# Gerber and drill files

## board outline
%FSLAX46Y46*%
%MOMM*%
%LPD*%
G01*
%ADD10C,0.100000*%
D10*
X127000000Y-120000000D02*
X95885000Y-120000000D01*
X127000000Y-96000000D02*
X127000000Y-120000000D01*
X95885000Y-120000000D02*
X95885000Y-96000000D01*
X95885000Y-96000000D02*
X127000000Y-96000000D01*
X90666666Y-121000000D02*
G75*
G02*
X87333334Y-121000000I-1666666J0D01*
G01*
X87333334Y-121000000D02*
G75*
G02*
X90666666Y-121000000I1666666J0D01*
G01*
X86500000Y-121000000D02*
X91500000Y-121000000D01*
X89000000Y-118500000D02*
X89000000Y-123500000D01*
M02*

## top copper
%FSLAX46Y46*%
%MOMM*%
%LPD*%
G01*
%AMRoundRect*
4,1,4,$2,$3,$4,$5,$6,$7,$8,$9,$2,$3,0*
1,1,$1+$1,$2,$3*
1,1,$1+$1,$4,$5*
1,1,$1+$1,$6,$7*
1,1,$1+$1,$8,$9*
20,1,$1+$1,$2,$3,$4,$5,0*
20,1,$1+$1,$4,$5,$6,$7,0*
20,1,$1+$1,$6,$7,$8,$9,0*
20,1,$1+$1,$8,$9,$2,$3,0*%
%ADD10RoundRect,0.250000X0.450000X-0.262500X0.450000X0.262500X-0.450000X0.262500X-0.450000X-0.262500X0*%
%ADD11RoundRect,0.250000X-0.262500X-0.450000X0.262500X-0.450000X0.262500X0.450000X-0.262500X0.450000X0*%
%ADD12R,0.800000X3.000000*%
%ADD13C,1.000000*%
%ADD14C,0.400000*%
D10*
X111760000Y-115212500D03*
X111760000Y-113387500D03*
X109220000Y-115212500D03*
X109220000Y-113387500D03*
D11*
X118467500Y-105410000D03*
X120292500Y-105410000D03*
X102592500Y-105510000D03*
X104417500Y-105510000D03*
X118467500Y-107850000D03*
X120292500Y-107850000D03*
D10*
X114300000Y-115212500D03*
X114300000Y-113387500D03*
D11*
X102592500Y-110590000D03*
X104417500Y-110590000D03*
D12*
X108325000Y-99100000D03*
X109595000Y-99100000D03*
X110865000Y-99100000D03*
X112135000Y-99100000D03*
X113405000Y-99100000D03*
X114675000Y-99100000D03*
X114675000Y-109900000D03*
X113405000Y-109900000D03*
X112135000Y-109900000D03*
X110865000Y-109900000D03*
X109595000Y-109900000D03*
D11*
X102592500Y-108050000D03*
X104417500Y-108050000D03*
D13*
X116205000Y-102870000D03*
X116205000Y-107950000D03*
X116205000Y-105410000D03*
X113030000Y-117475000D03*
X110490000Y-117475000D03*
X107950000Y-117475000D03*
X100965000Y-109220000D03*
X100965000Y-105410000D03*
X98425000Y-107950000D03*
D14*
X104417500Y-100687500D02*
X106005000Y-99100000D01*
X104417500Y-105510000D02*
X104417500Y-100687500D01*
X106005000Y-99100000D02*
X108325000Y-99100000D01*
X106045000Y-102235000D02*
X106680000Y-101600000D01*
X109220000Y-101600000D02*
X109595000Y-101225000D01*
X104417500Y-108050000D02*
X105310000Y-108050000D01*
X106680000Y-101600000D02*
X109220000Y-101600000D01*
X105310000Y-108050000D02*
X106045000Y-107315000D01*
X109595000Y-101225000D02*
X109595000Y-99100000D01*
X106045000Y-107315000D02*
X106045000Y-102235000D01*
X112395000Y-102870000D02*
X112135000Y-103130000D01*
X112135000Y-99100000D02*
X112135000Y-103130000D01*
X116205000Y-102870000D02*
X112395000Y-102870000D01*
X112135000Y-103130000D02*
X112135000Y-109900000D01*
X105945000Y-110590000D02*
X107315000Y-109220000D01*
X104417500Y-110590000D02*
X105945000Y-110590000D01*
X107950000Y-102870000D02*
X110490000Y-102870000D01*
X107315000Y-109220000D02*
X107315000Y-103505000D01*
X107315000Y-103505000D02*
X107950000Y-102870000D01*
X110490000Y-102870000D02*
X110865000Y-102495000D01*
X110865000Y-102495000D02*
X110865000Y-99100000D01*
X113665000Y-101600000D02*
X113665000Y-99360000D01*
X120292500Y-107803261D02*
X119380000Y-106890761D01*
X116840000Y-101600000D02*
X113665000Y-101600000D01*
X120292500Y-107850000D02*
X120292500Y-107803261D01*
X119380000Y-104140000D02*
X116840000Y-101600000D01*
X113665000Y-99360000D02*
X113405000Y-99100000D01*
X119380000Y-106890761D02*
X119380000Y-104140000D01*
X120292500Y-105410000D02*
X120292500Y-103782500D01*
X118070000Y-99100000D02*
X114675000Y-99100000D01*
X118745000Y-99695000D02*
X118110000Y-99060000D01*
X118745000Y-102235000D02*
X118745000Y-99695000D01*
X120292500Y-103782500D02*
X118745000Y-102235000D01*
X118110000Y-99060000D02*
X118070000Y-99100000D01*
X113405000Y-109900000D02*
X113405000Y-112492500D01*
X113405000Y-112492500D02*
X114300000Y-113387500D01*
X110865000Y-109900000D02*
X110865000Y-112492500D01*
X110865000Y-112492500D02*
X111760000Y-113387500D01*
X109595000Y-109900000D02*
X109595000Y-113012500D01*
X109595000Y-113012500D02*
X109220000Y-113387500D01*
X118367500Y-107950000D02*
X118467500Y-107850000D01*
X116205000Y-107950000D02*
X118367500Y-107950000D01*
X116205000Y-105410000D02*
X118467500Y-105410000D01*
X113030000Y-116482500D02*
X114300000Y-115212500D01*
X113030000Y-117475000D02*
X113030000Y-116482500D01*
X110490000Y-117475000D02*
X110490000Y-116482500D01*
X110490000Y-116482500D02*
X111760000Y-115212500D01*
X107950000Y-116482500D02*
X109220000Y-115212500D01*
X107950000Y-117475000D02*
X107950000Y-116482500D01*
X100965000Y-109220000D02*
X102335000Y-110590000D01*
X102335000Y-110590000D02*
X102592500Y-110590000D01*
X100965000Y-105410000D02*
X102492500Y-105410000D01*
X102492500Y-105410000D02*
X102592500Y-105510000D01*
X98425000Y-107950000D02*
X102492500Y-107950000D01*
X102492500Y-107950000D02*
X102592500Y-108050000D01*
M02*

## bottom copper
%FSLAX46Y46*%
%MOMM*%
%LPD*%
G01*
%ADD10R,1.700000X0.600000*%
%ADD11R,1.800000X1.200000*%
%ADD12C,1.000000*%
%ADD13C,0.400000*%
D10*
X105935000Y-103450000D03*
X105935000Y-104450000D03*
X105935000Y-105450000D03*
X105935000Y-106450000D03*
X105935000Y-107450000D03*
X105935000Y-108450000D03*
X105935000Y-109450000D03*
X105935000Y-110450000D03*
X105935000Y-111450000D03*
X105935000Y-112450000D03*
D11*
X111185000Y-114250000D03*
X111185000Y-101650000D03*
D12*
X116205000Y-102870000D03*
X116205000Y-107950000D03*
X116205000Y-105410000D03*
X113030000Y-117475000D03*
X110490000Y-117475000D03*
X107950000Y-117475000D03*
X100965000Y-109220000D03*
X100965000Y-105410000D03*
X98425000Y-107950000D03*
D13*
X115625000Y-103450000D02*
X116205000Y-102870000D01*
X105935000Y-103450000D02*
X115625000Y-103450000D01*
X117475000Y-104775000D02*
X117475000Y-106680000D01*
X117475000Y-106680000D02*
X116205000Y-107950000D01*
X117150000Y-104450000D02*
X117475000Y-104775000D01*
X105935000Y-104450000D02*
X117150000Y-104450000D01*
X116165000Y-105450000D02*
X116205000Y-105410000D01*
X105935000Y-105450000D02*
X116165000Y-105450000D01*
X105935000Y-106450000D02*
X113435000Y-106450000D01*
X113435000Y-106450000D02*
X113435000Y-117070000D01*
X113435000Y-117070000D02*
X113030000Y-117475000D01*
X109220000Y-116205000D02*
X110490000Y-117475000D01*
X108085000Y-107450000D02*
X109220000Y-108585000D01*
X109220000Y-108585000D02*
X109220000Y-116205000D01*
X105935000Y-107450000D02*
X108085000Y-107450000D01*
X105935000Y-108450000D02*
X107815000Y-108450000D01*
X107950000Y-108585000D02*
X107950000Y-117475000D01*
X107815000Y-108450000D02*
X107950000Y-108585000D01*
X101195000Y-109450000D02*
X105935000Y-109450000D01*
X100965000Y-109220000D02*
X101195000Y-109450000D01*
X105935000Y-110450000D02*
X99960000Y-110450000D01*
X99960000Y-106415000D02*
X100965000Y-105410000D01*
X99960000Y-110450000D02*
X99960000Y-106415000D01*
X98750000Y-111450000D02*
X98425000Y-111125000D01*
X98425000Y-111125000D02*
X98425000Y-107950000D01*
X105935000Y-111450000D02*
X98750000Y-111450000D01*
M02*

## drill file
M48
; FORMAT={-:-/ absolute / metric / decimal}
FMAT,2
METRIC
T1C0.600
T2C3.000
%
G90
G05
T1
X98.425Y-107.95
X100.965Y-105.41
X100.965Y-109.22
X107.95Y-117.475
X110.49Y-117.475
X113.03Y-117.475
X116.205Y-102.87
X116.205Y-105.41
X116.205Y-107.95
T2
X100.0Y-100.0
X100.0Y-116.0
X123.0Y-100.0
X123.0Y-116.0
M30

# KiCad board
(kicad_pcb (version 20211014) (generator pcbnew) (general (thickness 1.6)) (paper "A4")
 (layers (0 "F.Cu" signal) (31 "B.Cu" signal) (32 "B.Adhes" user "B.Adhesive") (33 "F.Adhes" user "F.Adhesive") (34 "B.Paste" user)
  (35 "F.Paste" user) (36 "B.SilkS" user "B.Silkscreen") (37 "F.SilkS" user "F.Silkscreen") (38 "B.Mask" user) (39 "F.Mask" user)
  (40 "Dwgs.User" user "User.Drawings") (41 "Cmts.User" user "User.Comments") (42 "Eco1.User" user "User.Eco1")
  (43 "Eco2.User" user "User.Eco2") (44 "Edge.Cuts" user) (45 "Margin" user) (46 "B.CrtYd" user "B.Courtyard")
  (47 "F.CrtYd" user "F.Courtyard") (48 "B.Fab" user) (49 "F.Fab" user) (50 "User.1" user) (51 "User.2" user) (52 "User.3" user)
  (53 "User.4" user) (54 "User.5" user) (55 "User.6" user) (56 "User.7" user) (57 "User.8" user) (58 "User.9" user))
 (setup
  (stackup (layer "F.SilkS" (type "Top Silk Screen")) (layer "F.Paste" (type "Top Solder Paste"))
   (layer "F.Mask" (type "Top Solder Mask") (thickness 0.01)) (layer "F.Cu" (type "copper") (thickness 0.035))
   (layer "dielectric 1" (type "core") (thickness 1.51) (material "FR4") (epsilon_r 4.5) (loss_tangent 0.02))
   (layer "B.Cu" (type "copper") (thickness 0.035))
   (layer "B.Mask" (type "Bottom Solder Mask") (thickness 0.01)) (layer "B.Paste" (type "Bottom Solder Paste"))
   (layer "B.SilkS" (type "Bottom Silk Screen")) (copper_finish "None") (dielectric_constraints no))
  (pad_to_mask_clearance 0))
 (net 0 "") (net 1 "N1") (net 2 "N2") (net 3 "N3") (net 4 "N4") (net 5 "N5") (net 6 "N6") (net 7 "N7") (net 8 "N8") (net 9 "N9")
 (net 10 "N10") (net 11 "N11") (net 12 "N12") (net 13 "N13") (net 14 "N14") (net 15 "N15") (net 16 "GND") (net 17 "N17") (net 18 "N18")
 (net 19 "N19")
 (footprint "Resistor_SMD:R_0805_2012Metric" (layer "F.Cu") (at 111.76 114.3 90)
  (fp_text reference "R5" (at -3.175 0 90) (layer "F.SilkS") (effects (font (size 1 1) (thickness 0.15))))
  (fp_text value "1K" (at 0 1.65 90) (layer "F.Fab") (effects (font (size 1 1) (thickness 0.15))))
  (pad "1" smd roundrect (at -0.9125 0 90) (size 1.025 1.4) (layers "F.Cu" "F.Paste" "F.Mask") (roundrect_rratio 0.243902) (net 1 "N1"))
  (pad "2" smd roundrect (at 0.9125 0 90) (size 1.025 1.4) (layers "F.Cu" "F.Paste" "F.Mask") (roundrect_rratio 0.243902) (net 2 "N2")))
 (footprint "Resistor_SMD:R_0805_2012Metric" (layer "F.Cu") (at 109.22 114.3 90)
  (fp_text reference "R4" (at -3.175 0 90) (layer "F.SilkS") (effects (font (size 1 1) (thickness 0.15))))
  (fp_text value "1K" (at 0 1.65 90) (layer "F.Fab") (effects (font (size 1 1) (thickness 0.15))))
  (pad "1" smd roundrect (at -0.9125 0 90) (size 1.025 1.4) (layers "F.Cu" "F.Paste" "F.Mask") (roundrect_rratio 0.243902) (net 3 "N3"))
  (pad "2" smd roundrect (at 0.9125 0 90) (size 1.025 1.4) (layers "F.Cu" "F.Paste" "F.Mask") (roundrect_rratio 0.243902) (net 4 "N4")))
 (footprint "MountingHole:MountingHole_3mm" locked (layer "F.Cu") (at 100 100)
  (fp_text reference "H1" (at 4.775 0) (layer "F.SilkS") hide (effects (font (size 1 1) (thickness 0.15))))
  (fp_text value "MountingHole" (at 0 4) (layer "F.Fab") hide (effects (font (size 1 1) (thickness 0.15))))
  (pad "" np_thru_hole circle locked (at 0 0) (size 3 3) (drill 3) (layers *.Cu *.Mask)))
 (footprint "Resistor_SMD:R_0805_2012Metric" (layer "F.Cu") (at 119.38 105.41)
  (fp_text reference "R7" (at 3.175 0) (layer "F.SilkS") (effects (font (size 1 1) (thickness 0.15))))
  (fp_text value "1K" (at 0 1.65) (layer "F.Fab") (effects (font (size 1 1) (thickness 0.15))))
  (pad "1" smd roundrect (at -0.9125 0) (size 1.025 1.4) (layers "F.Cu" "F.Paste" "F.Mask") (roundrect_rratio 0.243902) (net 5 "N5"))
  (pad "2" smd roundrect (at 0.9125 0) (size 1.025 1.4) (layers "F.Cu" "F.Paste" "F.Mask") (roundrect_rratio 0.243902) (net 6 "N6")))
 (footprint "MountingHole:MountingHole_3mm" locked (layer "F.Cu") (at 123 116)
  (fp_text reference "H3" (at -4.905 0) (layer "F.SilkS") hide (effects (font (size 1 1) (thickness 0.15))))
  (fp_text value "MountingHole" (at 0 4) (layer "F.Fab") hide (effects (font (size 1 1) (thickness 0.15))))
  (pad "" np_thru_hole circle locked (at 0 0) (size 3 3) (drill 3) (layers *.Cu *.Mask)))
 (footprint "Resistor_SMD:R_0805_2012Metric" (layer "F.Cu") (at 103.505 105.51)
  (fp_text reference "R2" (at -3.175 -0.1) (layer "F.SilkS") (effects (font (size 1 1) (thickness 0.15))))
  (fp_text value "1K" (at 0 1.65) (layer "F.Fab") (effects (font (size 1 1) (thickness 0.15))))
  (pad "1" smd roundrect (at -0.9125 0) (size 1.025 1.4) (layers "F.Cu" "F.Paste" "F.Mask") (roundrect_rratio 0.243902) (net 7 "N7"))
  (pad "2" smd roundrect (at 0.9125 0) (size 1.025 1.4) (layers "F.Cu" "F.Paste" "F.Mask") (roundrect_rratio 0.243902) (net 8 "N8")))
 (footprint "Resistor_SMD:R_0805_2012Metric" (layer "F.Cu") (at 119.38 107.85)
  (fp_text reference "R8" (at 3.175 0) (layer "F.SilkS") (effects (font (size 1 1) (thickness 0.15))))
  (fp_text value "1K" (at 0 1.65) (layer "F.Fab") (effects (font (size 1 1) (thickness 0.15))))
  (pad "1" smd roundrect (at -0.9125 0) (size 1.025 1.4) (layers "F.Cu" "F.Paste" "F.Mask") (roundrect_rratio 0.243902) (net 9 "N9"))
  (pad "2" smd roundrect (at 0.9125 0) (size 1.025 1.4) (layers "F.Cu" "F.Paste" "F.Mask") (roundrect_rratio 0.243902) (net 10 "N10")))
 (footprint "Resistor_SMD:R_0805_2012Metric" (layer "F.Cu") (at 114.3 114.3 90)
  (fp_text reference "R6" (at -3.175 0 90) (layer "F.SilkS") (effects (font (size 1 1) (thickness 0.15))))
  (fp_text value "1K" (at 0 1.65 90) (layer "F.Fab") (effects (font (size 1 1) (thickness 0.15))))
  (pad "1" smd roundrect (at -0.9125 0 90) (size 1.025 1.4) (layers "F.Cu" "F.Paste" "F.Mask") (roundrect_rratio 0.243902) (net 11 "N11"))
  (pad "2" smd roundrect (at 0.9125 0 90) (size 1.025 1.4) (layers "F.Cu" "F.Paste" "F.Mask") (roundrect_rratio 0.243902) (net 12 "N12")))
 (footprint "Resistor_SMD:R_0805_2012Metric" (layer "F.Cu") (at 103.505 110.59)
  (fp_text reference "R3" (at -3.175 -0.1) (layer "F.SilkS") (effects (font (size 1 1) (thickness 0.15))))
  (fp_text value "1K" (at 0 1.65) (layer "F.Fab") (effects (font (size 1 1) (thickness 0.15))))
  (pad "1" smd roundrect (at -0.9125 0) (size 1.025 1.4) (layers "F.Cu" "F.Paste" "F.Mask") (roundrect_rratio 0.243902) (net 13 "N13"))
  (pad "2" smd roundrect (at 0.9125 0) (size 1.025 1.4) (layers "F.Cu" "F.Paste" "F.Mask") (roundrect_rratio 0.243902) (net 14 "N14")))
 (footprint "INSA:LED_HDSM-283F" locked (layer "F.Cu") (at 111.5 104.5)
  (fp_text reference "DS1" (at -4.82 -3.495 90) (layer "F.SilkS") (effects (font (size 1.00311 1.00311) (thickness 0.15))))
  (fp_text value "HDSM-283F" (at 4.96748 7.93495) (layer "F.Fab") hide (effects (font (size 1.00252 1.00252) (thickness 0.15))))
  (pad "1" smd rect locked (at -3.175 -5.4 270) (size 3 0.8) (layers "F.Cu" "F.Paste" "F.Mask") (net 8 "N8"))
  (pad "2" smd rect locked (at -1.905 -5.4 270) (size 3 0.8) (layers "F.Cu" "F.Paste" "F.Mask") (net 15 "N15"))
  (pad "3" smd rect locked (at -0.635 -5.4 270) (size 3 0.8) (layers "F.Cu" "F.Paste" "F.Mask") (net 14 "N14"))
  (pad "4" smd rect locked (at 0.635 -5.4 270) (size 3 0.8) (layers "F.Cu" "F.Paste" "F.Mask") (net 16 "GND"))
  (pad "5" smd rect locked (at 1.905 -5.4 270) (size 3 0.8) (layers "F.Cu" "F.Paste" "F.Mask") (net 10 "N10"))
  (pad "6" smd rect locked (at 3.175 -5.4 270) (size 3 0.8) (layers "F.Cu" "F.Paste" "F.Mask") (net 6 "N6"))
  (pad "7" smd rect locked (at 3.175 5.4 270) (size 3 0.8) (layers "F.Cu" "F.Paste" "F.Mask") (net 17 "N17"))
  (pad "8" smd rect locked (at 1.905 5.4 270) (size 3 0.8) (layers "F.Cu" "F.Paste" "F.Mask") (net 12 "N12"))
  (pad "9" smd rect locked (at 0.635 5.4 270) (size 3 0.8) (layers "F.Cu" "F.Paste" "F.Mask") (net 16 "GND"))
  (pad "10" smd rect locked (at -0.635 5.4 270) (size 3 0.8) (layers "F.Cu" "F.Paste" "F.Mask") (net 2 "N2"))
  (pad "11" smd rect locked (at -1.905 5.4 270) (size 3 0.8) (layers "F.Cu" "F.Paste" "F.Mask") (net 4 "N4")))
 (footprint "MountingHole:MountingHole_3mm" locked (layer "F.Cu") (at 123 100)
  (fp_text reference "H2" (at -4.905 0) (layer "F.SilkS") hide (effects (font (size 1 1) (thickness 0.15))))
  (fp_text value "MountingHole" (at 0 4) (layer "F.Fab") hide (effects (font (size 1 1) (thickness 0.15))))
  (pad "" np_thru_hole circle locked (at 0 0) (size 3 3) (drill 3) (layers *.Cu *.Mask)))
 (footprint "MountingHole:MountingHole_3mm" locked (layer "F.Cu") (at 100 116)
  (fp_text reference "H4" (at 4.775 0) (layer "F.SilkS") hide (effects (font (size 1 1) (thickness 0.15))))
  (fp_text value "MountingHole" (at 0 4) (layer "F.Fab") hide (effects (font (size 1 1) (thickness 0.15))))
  (pad "" np_thru_hole circle locked (at 0 0) (size 3 3) (drill 3) (layers *.Cu *.Mask)))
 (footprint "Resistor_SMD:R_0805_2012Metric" (layer "F.Cu") (at 103.505 108.05)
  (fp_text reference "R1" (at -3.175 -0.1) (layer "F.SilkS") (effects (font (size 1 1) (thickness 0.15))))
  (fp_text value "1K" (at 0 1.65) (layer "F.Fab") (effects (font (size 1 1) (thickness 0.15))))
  (pad "1" smd roundrect (at -0.9125 0) (size 1.025 1.4) (layers "F.Cu" "F.Paste" "F.Mask") (roundrect_rratio 0.243902) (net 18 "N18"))
  (pad "2" smd roundrect (at 0.9125 0) (size 1.025 1.4) (layers "F.Cu" "F.Paste" "F.Mask") (roundrect_rratio 0.243902) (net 15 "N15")))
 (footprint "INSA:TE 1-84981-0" (layer "B.Cu") (at 106.285 107.95 -90)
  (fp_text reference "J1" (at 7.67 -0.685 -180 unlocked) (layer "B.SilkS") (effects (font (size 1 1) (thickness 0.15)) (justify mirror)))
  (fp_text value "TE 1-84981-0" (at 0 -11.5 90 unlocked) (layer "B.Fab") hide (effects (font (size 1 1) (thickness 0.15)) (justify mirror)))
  (pad "1" smd rect locked (at -4.5 0.35 270) (size 0.6 1.7) (layers "B.Cu" "B.Paste" "B.Mask") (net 16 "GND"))
  (pad "2" smd rect locked (at -3.5 0.35 270) (size 0.6 1.7) (layers "B.Cu" "B.Paste" "B.Mask") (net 9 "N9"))
  (pad "3" smd rect locked (at -2.5 0.35 270) (size 0.6 1.7) (layers "B.Cu" "B.Paste" "B.Mask") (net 5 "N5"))
  (pad "4" smd rect locked (at -1.5 0.35 270) (size 0.6 1.7) (layers "B.Cu" "B.Paste" "B.Mask") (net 11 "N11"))
  (pad "5" smd rect locked (at -0.5 0.35 270) (size 0.6 1.7) (layers "B.Cu" "B.Paste" "B.Mask") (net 1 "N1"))
  (pad "6" smd rect locked (at 0.5 0.35 270) (size 0.6 1.7) (layers "B.Cu" "B.Paste" "B.Mask") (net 3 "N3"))
  (pad "7" smd rect locked (at 1.5 0.35 270) (size 0.6 1.7) (layers "B.Cu" "B.Paste" "B.Mask") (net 13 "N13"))
  (pad "8" smd rect locked (at 2.5 0.35 270) (size 0.6 1.7) (layers "B.Cu" "B.Paste" "B.Mask") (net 7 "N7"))
  (pad "9" smd rect locked (at 3.5 0.35 270) (size 0.6 1.7) (layers "B.Cu" "B.Paste" "B.Mask") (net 18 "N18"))
  (pad "10" smd rect locked (at 4.5 0.35 270) (size 0.6 1.7) (layers "B.Cu" "B.Paste" "B.Mask") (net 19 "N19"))
  (pad "11" smd rect locked (at 6.3 -4.9 270) (size 1.2 1.8) (layers "B.Cu" "B.Paste" "B.Mask"))
  (pad "11" smd rect locked (at -6.3 -4.9 270) (size 1.2 1.8) (layers "B.Cu" "B.Paste" "B.Mask")))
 (gr_line (start 127 120) (end 95.885 120) (layer "Edge.Cuts") (width 0.1))
 (gr_line (start 127 96) (end 127 120) (layer "Edge.Cuts") (width 0.1))
 (gr_line (start 95.885 120) (end 95.885 96) (layer "Edge.Cuts") (width 0.1))
 (gr_line (start 95.885 96) (end 127 96) (layer "Edge.Cuts") (width 0.1))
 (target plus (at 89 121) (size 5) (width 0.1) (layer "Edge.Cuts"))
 (segment (start 104.4175 100.6875) (end 106.005 99.1) (width 0.4) (layer "F.Cu") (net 8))
 (segment (start 104.4175 105.51) (end 104.4175 100.6875) (width 0.4) (layer "F.Cu") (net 8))
 (segment (start 106.005 99.1) (end 108.325 99.1) (width 0.4) (layer "F.Cu") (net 8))
 (segment (start 106.045 102.235) (end 106.68 101.6) (width 0.4) (layer "F.Cu") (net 15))
 (segment (start 109.22 101.6) (end 109.595 101.225) (width 0.4) (layer "F.Cu") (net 15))
 (segment (start 104.4175 108.05) (end 105.31 108.05) (width 0.4) (layer "F.Cu") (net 15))
 (segment (start 106.68 101.6) (end 109.22 101.6) (width 0.4) (layer "F.Cu") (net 15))
 (segment (start 105.31 108.05) (end 106.045 107.315) (width 0.4) (layer "F.Cu") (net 15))
 (segment (start 109.595 101.225) (end 109.595 99.1) (width 0.4) (layer "F.Cu") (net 15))
 (segment (start 106.045 107.315) (end 106.045 102.235) (width 0.4) (layer "F.Cu") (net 15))
 (segment (start 112.395 102.87) (end 112.135 103.13) (width 0.4) (layer "F.Cu") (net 16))
 (segment (start 112.135 99.1) (end 112.135 103.13) (width 0.4) (layer "F.Cu") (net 16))
 (segment (start 116.205 102.87) (end 112.395 102.87) (width 0.4) (layer "F.Cu") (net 16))
 (segment (start 112.135 103.13) (end 112.135 109.9) (width 0.4) (layer "F.Cu") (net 16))
 (via (at 116.205 102.87) (size 1) (drill 0.6) (layers "F.Cu" "B.Cu") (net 16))
 (segment (start 115.625 103.45) (end 116.205 102.87) (width 0.4) (layer "B.Cu") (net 16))
 (segment (start 105.935 103.45) (end 115.625 103.45) (width 0.4) (layer "B.Cu") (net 16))
 (segment (start 105.945 110.59) (end 107.315 109.22) (width 0.4) (layer "F.Cu") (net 14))
 (segment (start 104.4175 110.59) (end 105.945 110.59) (width 0.4) (layer "F.Cu") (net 14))
 (segment (start 107.95 102.87) (end 110.49 102.87) (width 0.4) (layer "F.Cu") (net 14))
 (segment (start 107.315 109.22) (end 107.315 103.505) (width 0.4) (layer "F.Cu") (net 14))
 (segment (start 107.315 103.505) (end 107.95 102.87) (width 0.4) (layer "F.Cu") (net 14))
 (segment (start 110.49 102.87) (end 110.865 102.495) (width 0.4) (layer "F.Cu") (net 14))
 (segment (start 110.865 102.495) (end 110.865 99.1) (width 0.4) (layer "F.Cu") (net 14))
 (segment (start 113.665 101.6) (end 113.665 99.36) (width 0.4) (layer "F.Cu") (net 10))
 (segment (start 120.2925 107.803261) (end 119.38 106.890761) (width 0.4) (layer "F.Cu") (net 10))
 (segment (start 116.84 101.6) (end 113.665 101.6) (width 0.4) (layer "F.Cu") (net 10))
 (segment (start 120.2925 107.85) (end 120.2925 107.803261) (width 0.4) (layer "F.Cu") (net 10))
 (segment (start 119.38 104.14) (end 116.84 101.6) (width 0.4) (layer "F.Cu") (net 10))
 (segment (start 113.665 99.36) (end 113.405 99.1) (width 0.4) (layer "F.Cu") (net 10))
 (segment (start 119.38 106.890761) (end 119.38 104.14) (width 0.4) (layer "F.Cu") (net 10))
 (segment (start 120.2925 105.41) (end 120.2925 103.7825) (width 0.4) (layer "F.Cu") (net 6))
 (segment (start 118.07 99.1) (end 114.675 99.1) (width 0.4) (layer "F.Cu") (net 6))
 (segment (start 118.745 99.695) (end 118.11 99.06) (width 0.4) (layer "F.Cu") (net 6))
 (segment (start 118.745 102.235) (end 118.745 99.695) (width 0.4) (layer "F.Cu") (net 6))
 (segment (start 120.2925 103.7825) (end 118.745 102.235) (width 0.4) (layer "F.Cu") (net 6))
 (segment (start 118.11 99.06) (end 118.07 99.1) (width 0.4) (layer "F.Cu") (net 6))
 (segment (start 113.405 109.9) (end 113.405 112.4925) (width 0.4) (layer "F.Cu") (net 12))
 (segment (start 113.405 112.4925) (end 114.3 113.3875) (width 0.4) (layer "F.Cu") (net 12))
 (segment (start 110.865 109.9) (end 110.865 112.4925) (width 0.4) (layer "F.Cu") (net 2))
 (segment (start 110.865 112.4925) (end 111.76 113.3875) (width 0.4) (layer "F.Cu") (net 2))
 (segment (start 109.595 109.9) (end 109.595 113.0125) (width 0.4) (layer "F.Cu") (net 4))
 (segment (start 109.595 113.0125) (end 109.22 113.3875) (width 0.4) (layer "F.Cu") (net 4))
 (segment (start 118.3675 107.95) (end 118.4675 107.85) (width 0.4) (layer "F.Cu") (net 9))
 (segment (start 116.205 107.95) (end 118.3675 107.95) (width 0.4) (layer "F.Cu") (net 9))
 (via (at 116.205 107.95) (size 1) (drill 0.6) (layers "F.Cu" "B.Cu") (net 9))
 (segment (start 117.475 104.775) (end 117.475 106.68) (width 0.4) (layer "B.Cu") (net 9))
 (segment (start 117.475 106.68) (end 116.205 107.95) (width 0.4) (layer "B.Cu") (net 9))
 (segment (start 117.15 104.45) (end 117.475 104.775) (width 0.4) (layer "B.Cu") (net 9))
 (segment (start 105.935 104.45) (end 117.15 104.45) (width 0.4) (layer "B.Cu") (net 9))
 (segment (start 116.205 105.41) (end 118.4675 105.41) (width 0.4) (layer "F.Cu") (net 5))
 (via (at 116.205 105.41) (size 1) (drill 0.6) (layers "F.Cu" "B.Cu") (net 5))
 (segment (start 116.165 105.45) (end 116.205 105.41) (width 0.4) (layer "B.Cu") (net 5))
 (segment (start 105.935 105.45) (end 116.165 105.45) (width 0.4) (layer "B.Cu") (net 5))
 (segment (start 113.03 116.4825) (end 114.3 115.2125) (width 0.4) (layer "F.Cu") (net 11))
 (segment (start 113.03 117.475) (end 113.03 116.4825) (width 0.4) (layer "F.Cu") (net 11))
 (via (at 113.03 117.475) (size 1) (drill 0.6) (layers "F.Cu" "B.Cu") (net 11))
 (segment (start 105.935 106.45) (end 113.435 106.45) (width 0.4) (layer "B.Cu") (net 11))
 (segment (start 113.435 106.45) (end 113.435 117.07) (width 0.4) (layer "B.Cu") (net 11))
 (segment (start 113.435 117.07) (end 113.03 117.475) (width 0.4) (layer "B.Cu") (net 11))
 (segment (start 110.49 117.475) (end 110.49 116.4825) (width 0.4) (layer "F.Cu") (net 1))
 (segment (start 110.49 116.4825) (end 111.76 115.2125) (width 0.4) (layer "F.Cu") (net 1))
 (via (at 110.49 117.475) (size 1) (drill 0.6) (layers "F.Cu" "B.Cu") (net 1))
 (segment (start 109.22 116.205) (end 110.49 117.475) (width 0.4) (layer "B.Cu") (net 1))
 (segment (start 108.085 107.45) (end 109.22 108.585) (width 0.4) (layer "B.Cu") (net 1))
 (segment (start 109.22 108.585) (end 109.22 116.205) (width 0.4) (layer "B.Cu") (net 1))
 (segment (start 105.935 107.45) (end 108.085 107.45) (width 0.4) (layer "B.Cu") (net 1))
 (segment (start 107.95 116.4825) (end 109.22 115.2125) (width 0.4) (layer "F.Cu") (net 3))
 (segment (start 107.95 117.475) (end 107.95 116.4825) (width 0.4) (layer "F.Cu") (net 3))
 (via (at 107.95 117.475) (size 1) (drill 0.6) (layers "F.Cu" "B.Cu") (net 3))
 (segment (start 105.935 108.45) (end 107.815 108.45) (width 0.4) (layer "B.Cu") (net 3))
 (segment (start 107.95 108.585) (end 107.95 117.475) (width 0.4) (layer "B.Cu") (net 3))
 (segment (start 107.815 108.45) (end 107.95 108.585) (width 0.4) (layer "B.Cu") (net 3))
 (segment (start 100.965 109.22) (end 102.335 110.59) (width 0.4) (layer "F.Cu") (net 13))
 (segment (start 102.335 110.59) (end 102.5925 110.59) (width 0.4) (layer "F.Cu") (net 13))
 (via (at 100.965 109.22) (size 1) (drill 0.6) (layers "F.Cu" "B.Cu") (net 13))
 (segment (start 101.195 109.45) (end 105.935 109.45) (width 0.4) (layer "B.Cu") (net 13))
 (segment (start 100.965 109.22) (end 101.195 109.45) (width 0.4) (layer "B.Cu") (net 13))
 (segment (start 100.965 105.41) (end 102.4925 105.41) (width 0.4) (layer "F.Cu") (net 7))
 (segment (start 102.4925 105.41) (end 102.5925 105.51) (width 0.4) (layer "F.Cu") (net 7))
 (via (at 100.965 105.41) (size 1) (drill 0.6) (layers "F.Cu" "B.Cu") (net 7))
 (segment (start 105.935 110.45) (end 99.96 110.45) (width 0.4) (layer "B.Cu") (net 7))
 (segment (start 99.96 106.415) (end 100.965 105.41) (width 0.4) (layer "B.Cu") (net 7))
 (segment (start 99.96 110.45) (end 99.96 106.415) (width 0.4) (layer "B.Cu") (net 7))
 (segment (start 98.425 107.95) (end 102.4925 107.95) (width 0.4) (layer "F.Cu") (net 18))
 (segment (start 102.4925 107.95) (end 102.5925 108.05) (width 0.4) (layer "F.Cu") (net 18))
 (via (at 98.425 107.95) (size 1) (drill 0.6) (layers "F.Cu" "B.Cu") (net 18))
 (segment (start 98.75 111.45) (end 98.425 111.125) (width 0.4) (layer "B.Cu") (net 18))
 (segment (start 98.425 111.125) (end 98.425 107.95) (width 0.4) (layer "B.Cu") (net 18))
 (segment (start 105.935 111.45) (end 98.75 111.45) (width 0.4) (layer "B.Cu") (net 18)))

